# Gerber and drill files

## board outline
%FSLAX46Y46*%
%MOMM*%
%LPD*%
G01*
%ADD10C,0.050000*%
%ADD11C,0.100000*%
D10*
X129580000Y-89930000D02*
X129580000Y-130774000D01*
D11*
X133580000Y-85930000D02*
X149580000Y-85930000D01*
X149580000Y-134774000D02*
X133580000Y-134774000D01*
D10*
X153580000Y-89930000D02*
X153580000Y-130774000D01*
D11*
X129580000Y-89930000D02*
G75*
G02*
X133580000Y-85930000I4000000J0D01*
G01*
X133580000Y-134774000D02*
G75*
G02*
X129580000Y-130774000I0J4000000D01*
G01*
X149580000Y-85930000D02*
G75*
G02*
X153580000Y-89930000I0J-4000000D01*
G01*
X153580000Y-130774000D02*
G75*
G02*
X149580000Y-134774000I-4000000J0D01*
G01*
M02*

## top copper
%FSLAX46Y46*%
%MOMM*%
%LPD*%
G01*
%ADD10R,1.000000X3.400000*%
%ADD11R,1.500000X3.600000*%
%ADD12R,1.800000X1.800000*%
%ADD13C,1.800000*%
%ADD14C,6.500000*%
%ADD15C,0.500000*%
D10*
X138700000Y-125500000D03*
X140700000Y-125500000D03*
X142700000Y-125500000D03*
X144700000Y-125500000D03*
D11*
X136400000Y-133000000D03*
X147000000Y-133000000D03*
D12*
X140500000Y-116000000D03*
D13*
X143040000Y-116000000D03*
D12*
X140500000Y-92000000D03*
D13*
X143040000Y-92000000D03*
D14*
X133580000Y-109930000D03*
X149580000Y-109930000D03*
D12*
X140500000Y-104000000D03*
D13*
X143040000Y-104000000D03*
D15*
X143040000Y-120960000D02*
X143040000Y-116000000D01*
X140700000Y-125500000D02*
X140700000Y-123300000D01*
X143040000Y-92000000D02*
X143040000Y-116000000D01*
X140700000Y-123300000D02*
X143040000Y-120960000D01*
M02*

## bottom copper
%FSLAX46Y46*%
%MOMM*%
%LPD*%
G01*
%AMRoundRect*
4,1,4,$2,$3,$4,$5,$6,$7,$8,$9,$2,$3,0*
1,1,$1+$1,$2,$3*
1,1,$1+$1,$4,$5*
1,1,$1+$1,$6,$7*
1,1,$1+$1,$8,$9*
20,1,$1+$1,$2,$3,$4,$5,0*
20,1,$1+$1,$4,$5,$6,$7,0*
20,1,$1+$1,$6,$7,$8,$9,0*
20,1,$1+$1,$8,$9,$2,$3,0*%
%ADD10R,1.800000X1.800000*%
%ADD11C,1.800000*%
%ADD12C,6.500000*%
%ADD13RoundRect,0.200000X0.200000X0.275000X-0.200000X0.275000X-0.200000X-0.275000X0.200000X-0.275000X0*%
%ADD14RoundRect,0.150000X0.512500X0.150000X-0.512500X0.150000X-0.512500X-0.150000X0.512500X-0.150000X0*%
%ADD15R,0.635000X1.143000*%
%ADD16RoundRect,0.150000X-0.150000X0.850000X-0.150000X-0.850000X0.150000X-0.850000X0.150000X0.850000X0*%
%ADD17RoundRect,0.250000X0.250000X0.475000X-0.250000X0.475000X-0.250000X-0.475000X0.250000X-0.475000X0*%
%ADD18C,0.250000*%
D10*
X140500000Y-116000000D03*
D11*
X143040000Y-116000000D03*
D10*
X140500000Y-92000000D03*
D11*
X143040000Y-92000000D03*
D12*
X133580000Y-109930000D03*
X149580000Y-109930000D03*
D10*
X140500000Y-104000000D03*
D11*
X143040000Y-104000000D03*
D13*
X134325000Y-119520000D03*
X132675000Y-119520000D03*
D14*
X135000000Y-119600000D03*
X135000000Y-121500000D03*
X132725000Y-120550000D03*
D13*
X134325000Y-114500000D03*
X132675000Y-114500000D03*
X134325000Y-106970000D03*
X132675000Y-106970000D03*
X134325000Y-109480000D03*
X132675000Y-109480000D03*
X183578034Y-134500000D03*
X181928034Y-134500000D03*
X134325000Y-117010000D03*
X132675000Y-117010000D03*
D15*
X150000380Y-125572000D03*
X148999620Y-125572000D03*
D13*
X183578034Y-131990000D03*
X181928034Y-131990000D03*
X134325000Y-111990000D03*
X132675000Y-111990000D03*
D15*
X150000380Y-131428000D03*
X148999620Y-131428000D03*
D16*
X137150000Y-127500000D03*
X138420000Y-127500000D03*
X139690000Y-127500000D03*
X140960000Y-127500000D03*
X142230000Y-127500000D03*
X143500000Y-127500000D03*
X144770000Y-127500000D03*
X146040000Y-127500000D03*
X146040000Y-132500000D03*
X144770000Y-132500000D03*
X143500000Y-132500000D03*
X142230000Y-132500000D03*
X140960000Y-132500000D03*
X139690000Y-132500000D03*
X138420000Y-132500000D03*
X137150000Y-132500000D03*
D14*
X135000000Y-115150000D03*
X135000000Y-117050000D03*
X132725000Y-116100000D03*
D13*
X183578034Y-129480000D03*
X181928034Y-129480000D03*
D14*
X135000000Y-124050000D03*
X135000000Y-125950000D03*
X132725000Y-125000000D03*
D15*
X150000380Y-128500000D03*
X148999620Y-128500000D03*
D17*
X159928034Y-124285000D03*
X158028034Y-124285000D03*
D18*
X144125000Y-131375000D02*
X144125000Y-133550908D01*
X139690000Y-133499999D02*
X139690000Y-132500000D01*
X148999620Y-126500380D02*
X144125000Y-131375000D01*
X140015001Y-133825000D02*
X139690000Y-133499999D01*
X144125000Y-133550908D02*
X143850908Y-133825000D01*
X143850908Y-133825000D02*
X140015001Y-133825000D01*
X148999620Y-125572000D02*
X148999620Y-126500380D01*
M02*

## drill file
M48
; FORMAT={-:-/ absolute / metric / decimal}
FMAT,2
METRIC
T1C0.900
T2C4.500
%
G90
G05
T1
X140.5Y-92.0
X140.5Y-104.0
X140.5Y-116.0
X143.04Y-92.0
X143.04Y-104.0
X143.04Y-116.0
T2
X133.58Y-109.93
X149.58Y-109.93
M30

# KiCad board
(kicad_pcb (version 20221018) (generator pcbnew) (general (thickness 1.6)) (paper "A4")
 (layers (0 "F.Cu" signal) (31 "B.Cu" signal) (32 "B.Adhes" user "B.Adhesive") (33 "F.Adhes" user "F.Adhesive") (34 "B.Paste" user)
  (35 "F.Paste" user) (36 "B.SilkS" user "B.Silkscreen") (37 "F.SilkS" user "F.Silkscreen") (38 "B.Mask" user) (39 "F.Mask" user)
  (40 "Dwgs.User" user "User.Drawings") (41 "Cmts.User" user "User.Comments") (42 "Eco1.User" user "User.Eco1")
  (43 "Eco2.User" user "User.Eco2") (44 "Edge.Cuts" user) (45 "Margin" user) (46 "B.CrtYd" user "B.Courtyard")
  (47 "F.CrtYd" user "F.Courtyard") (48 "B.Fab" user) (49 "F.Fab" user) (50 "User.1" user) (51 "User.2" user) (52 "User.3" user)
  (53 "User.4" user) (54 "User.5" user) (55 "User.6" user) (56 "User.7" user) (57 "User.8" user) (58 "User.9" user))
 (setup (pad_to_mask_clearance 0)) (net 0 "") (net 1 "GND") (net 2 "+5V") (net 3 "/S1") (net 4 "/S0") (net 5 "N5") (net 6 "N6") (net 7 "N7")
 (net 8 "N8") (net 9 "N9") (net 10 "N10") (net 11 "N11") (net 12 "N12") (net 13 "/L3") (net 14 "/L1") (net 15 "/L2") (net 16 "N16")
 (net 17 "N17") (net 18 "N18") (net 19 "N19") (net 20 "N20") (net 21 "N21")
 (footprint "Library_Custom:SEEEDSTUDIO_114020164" (layer "F.Cu") (at 141.7 129.825)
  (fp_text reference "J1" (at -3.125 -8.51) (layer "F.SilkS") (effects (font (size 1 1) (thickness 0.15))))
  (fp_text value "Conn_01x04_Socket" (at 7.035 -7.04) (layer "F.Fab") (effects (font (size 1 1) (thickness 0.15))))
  (pad "1" smd rect (at -3 -4.325) (size 1 3.4) (layers "F.Cu" "F.Paste" "F.Mask") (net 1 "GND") (solder_mask_margin 0.102))
  (pad "2" smd rect (at -1 -4.325) (size 1 3.4) (layers "F.Cu" "F.Paste" "F.Mask") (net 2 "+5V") (solder_mask_margin 0.102))
  (pad "3" smd rect (at 1 -4.325) (size 1 3.4) (layers "F.Cu" "F.Paste" "F.Mask") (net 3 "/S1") (solder_mask_margin 0.102))
  (pad "4" smd rect (at 3 -4.325) (size 1 3.4) (layers "F.Cu" "F.Paste" "F.Mask") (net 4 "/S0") (solder_mask_margin 0.102))
  (pad "SH1" smd rect (at -5.3 3.175) (size 1.5 3.6) (layers "F.Cu" "F.Paste" "F.Mask") (solder_mask_margin 0.102))
  (pad "SH2" smd rect (at 5.3 3.175) (size 1.5 3.6) (layers "F.Cu" "F.Paste" "F.Mask") (solder_mask_margin 0.102)))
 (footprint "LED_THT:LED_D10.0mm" (layer "F.Cu") (at 140.5 116)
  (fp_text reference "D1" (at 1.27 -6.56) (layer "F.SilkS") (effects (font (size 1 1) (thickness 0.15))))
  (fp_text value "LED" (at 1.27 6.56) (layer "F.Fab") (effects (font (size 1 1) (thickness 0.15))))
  (pad "1" thru_hole rect (at 0 0) (size 1.8 1.8) (drill 0.9) (layers "*.Cu" "*.Mask") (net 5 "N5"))
  (pad "2" thru_hole circle (at 2.54 0) (size 1.8 1.8) (drill 0.9) (layers "*.Cu" "*.Mask") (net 2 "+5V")))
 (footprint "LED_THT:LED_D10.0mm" (layer "F.Cu") (at 140.5 92)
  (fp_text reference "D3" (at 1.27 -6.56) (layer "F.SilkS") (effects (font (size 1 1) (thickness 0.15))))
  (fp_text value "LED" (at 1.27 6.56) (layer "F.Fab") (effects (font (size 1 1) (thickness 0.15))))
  (pad "1" thru_hole rect (at 0 0) (size 1.8 1.8) (drill 0.9) (layers "*.Cu" "*.Mask") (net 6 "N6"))
  (pad "2" thru_hole circle (at 2.54 0) (size 1.8 1.8) (drill 0.9) (layers "*.Cu" "*.Mask") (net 2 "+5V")))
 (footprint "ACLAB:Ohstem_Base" (layer "F.Cu") (at 142.5 116)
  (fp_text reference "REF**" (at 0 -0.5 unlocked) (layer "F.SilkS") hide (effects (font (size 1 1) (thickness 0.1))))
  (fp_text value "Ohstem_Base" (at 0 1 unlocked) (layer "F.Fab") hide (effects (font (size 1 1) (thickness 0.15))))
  (fp_line (start -12.92 -26.07) (end -12.92 14.774) (stroke (width 0.05) (type default)) (layer "Edge.Cuts"))
  (fp_line (start -8.92 -30.07) (end 7.08 -30.07) (stroke (width 0.1) (type default)) (layer "Edge.Cuts"))
  (fp_line (start 7.08 18.774) (end -8.92 18.774) (stroke (width 0.1) (type default)) (layer "Edge.Cuts"))
  (fp_line (start 11.08 -26.07) (end 11.08 14.774) (stroke (width 0.05) (type default)) (layer "Edge.Cuts"))
  (fp_arc (start -12.92 -26.07) (mid -11.748427 -28.898427) (end -8.92 -30.07) (stroke (width 0.1) (type default)) (layer "Edge.Cuts"))
  (fp_arc (start -8.92 18.774) (mid -11.748427 17.602427) (end -12.92 14.774) (stroke (width 0.1) (type default)) (layer "Edge.Cuts"))
  (fp_arc (start 7.08 -30.07) (mid 9.908427 -28.898427) (end 11.08 -26.07) (stroke (width 0.1) (type default)) (layer "Edge.Cuts"))
  (fp_arc (start 11.08 14.774) (mid 9.908427 17.602427) (end 7.08 18.774) (stroke (width 0.1) (type default)) (layer "Edge.Cuts"))
  (pad "1" thru_hole circle (at -8.92 -6.07) (size 6.5 6.5) (drill 4.5) (layers "*.Cu" "*.Mask"))
  (pad "1" thru_hole circle (at 7.08 -6.07) (size 6.5 6.5) (drill 4.5) (layers "*.Cu" "*.Mask")))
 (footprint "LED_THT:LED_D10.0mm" (layer "F.Cu") (at 140.5 104)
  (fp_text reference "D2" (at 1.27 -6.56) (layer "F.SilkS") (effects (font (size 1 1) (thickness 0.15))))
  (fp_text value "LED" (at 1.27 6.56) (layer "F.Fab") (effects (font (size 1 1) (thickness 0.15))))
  (pad "1" thru_hole rect (at 0 0) (size 1.8 1.8) (drill 0.9) (layers "*.Cu" "*.Mask") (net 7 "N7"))
  (pad "2" thru_hole circle (at 2.54 0) (size 1.8 1.8) (drill 0.9) (layers "*.Cu" "*.Mask") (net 2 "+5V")))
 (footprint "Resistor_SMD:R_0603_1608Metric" (layer "B.Cu") (at 133.5 119.52 180)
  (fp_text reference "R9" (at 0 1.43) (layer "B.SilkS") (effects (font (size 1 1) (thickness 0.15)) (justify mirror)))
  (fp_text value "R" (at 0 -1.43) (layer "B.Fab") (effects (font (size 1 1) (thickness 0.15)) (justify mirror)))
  (pad "1" smd roundrect (at -0.825 0 180) (size 0.8 0.95) (layers "B.Cu" "B.Paste" "B.Mask") (roundrect_rratio 0.25) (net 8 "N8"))
  (pad "2" smd roundrect (at 0.825 0 180) (size 0.8 0.95) (layers "B.Cu" "B.Paste" "B.Mask") (roundrect_rratio 0.25) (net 1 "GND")))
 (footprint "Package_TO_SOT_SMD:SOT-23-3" (layer "B.Cu") (at 133.8625 120.55 180)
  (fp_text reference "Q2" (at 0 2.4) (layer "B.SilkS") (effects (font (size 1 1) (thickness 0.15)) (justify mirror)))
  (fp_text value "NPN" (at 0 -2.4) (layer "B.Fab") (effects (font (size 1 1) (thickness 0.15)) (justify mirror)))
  (pad "1" smd roundrect (at -1.1375 0.95 180) (size 1.325 0.6) (layers "B.Cu" "B.Paste" "B.Mask") (roundrect_rratio 0.25) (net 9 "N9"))
  (pad "2" smd roundrect (at -1.1375 -0.95 180) (size 1.325 0.6) (layers "B.Cu" "B.Paste" "B.Mask") (roundrect_rratio 0.25) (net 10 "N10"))
  (pad "3" smd roundrect (at 1.1375 0 180) (size 1.325 0.6) (layers "B.Cu" "B.Paste" "B.Mask") (roundrect_rratio 0.25) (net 1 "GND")))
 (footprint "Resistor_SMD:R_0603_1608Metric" (layer "B.Cu") (at 133.5 114.5 180)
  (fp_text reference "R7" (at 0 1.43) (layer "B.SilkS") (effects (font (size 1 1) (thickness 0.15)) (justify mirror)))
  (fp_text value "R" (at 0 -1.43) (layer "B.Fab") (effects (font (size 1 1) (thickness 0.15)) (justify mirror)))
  (pad "1" smd roundrect (at -0.825 0 180) (size 0.8 0.95) (layers "B.Cu" "B.Paste" "B.Mask") (roundrect_rratio 0.25) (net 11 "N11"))
  (pad "2" smd roundrect (at 0.825 0 180) (size 0.8 0.95) (layers "B.Cu" "B.Paste" "B.Mask") (roundrect_rratio 0.25) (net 1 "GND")))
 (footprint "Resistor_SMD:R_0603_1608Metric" (layer "B.Cu") (at 133.5 106.97 180)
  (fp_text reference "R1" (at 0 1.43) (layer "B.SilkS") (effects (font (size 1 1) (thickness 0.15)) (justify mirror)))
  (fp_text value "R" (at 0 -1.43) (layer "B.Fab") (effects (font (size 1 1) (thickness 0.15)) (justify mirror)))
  (pad "1" smd roundrect (at -0.825 0 180) (size 0.8 0.95) (layers "B.Cu" "B.Paste" "B.Mask") (roundrect_rratio 0.25) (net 5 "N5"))
  (pad "2" smd roundrect (at 0.825 0 180) (size 0.8 0.95) (layers "B.Cu" "B.Paste" "B.Mask") (roundrect_rratio 0.25) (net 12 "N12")))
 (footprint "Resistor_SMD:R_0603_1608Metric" (layer "B.Cu") (at 133.5 109.48 180)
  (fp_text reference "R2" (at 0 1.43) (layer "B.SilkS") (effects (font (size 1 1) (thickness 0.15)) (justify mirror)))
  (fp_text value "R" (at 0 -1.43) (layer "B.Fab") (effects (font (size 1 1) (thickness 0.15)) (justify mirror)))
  (pad "1" smd roundrect (at -0.825 0 180) (size 0.8 0.95) (layers "B.Cu" "B.Paste" "B.Mask") (roundrect_rratio 0.25) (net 7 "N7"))
  (pad "2" smd roundrect (at 0.825 0 180) (size 0.8 0.95) (layers "B.Cu" "B.Paste" "B.Mask") (roundrect_rratio 0.25) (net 9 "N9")))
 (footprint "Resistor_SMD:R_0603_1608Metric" (layer "B.Cu") (at 182.753034 134.5 180)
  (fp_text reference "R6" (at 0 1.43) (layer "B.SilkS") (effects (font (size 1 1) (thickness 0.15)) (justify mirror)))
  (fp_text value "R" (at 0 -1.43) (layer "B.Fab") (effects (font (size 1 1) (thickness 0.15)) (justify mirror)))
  (pad "1" smd roundrect (at -0.825 0 180) (size 0.8 0.95) (layers "B.Cu" "B.Paste" "B.Mask") (roundrect_rratio 0.25) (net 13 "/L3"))
  (pad "2" smd roundrect (at 0.825 0 180) (size 0.8 0.95) (layers "B.Cu" "B.Paste" "B.Mask") (roundrect_rratio 0.25) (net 8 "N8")))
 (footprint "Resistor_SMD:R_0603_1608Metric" (layer "B.Cu") (at 133.5 117.01 180)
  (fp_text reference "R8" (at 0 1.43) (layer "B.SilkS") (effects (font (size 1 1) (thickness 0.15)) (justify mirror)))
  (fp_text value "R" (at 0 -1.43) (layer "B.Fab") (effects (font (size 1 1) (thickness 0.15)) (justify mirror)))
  (pad "1" smd roundrect (at -0.825 0 180) (size 0.8 0.95) (layers "B.Cu" "B.Paste" "B.Mask") (roundrect_rratio 0.25) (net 10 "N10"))
  (pad "2" smd roundrect (at 0.825 0 180) (size 0.8 0.95) (layers "B.Cu" "B.Paste" "B.Mask") (roundrect_rratio 0.25) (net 1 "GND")))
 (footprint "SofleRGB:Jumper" (layer "B.Cu") (at 149.5 125.572 180)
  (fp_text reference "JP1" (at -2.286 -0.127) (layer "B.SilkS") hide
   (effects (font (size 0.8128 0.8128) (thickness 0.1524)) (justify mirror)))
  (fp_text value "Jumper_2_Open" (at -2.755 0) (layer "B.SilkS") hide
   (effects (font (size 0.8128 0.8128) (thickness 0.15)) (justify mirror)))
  (pad "1" smd rect (at -0.50038 0 180) (size 0.635 1.143) (layers "B.Cu" "B.Paste" "B.Mask") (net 12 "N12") (clearance 0.1905))
  (pad "2" smd rect (at 0.50038 0 180) (size 0.635 1.143) (layers "B.Cu" "B.Paste" "B.Mask") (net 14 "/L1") (clearance 0.1905)))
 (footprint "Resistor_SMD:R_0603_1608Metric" (layer "B.Cu") (at 182.753034 131.99 180)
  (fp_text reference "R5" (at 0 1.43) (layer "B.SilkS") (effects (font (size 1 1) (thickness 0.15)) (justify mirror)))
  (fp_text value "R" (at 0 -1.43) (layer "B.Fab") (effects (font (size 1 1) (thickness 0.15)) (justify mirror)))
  (pad "1" smd roundrect (at -0.825 0 180) (size 0.8 0.95) (layers "B.Cu" "B.Paste" "B.Mask") (roundrect_rratio 0.25) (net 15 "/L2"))
  (pad "2" smd roundrect (at 0.825 0 180) (size 0.8 0.95) (layers "B.Cu" "B.Paste" "B.Mask") (roundrect_rratio 0.25) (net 10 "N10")))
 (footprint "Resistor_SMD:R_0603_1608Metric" (layer "B.Cu") (at 133.5 111.99 180)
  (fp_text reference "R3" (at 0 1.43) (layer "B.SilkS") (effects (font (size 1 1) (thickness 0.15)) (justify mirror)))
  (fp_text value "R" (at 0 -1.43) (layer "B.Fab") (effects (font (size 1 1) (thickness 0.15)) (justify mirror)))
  (pad "1" smd roundrect (at -0.825 0 180) (size 0.8 0.95) (layers "B.Cu" "B.Paste" "B.Mask") (roundrect_rratio 0.25) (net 6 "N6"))
  (pad "2" smd roundrect (at 0.825 0 180) (size 0.8 0.95) (layers "B.Cu" "B.Paste" "B.Mask") (roundrect_rratio 0.25) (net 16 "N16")))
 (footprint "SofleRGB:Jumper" (layer "B.Cu") (at 149.5 131.428 180)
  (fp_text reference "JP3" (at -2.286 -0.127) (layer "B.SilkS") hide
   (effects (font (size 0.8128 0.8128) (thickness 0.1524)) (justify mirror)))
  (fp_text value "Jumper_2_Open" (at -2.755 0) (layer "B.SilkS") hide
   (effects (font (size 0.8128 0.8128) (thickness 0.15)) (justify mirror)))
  (pad "1" smd rect (at -0.50038 0 180) (size 0.635 1.143) (layers "B.Cu" "B.Paste" "B.Mask") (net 13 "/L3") (clearance 0.1905))
  (pad "2" smd rect (at 0.50038 0 180) (size 0.635 1.143) (layers "B.Cu" "B.Paste" "B.Mask") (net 16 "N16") (clearance 0.1905)))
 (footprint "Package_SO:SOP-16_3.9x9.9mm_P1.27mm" (layer "B.Cu") (at 141.595 130 -90)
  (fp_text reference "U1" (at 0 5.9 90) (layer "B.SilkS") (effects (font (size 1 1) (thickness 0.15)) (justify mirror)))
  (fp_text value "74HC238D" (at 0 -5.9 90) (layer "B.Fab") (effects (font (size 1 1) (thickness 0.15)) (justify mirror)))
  (pad "1" smd roundrect (at -2.5 4.445 270) (size 2 0.6) (layers "B.Cu" "B.Paste" "B.Mask") (roundrect_rratio 0.25) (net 4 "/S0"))
  (pad "2" smd roundrect (at -2.5 3.175 270) (size 2 0.6) (layers "B.Cu" "B.Paste" "B.Mask") (roundrect_rratio 0.25) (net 3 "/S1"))
  (pad "3" smd roundrect (at -2.5 1.905 270) (size 2 0.6) (layers "B.Cu" "B.Paste" "B.Mask") (roundrect_rratio 0.25) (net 1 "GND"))
  (pad "4" smd roundrect (at -2.5 0.635 270) (size 2 0.6) (layers "B.Cu" "B.Paste" "B.Mask") (roundrect_rratio 0.25) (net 1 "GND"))
  (pad "5" smd roundrect (at -2.5 -0.635 270) (size 2 0.6) (layers "B.Cu" "B.Paste" "B.Mask") (roundrect_rratio 0.25) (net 1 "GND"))
  (pad "6" smd roundrect (at -2.5 -1.905 270) (size 2 0.6) (layers "B.Cu" "B.Paste" "B.Mask") (roundrect_rratio 0.25) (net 2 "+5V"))
  (pad "7" smd roundrect (at -2.5 -3.175 270) (size 2 0.6) (layers "B.Cu" "B.Paste" "B.Mask") (roundrect_rratio 0.25) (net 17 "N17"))
  (pad "8" smd roundrect (at -2.5 -4.445 270) (size 2 0.6) (layers "B.Cu" "B.Paste" "B.Mask") (roundrect_rratio 0.25) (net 1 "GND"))
  (pad "9" smd roundrect (at 2.5 -4.445 270) (size 2 0.6) (layers "B.Cu" "B.Paste" "B.Mask") (roundrect_rratio 0.25) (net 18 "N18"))
  (pad "10" smd roundrect (at 2.5 -3.175 270) (size 2 0.6) (layers "B.Cu" "B.Paste" "B.Mask") (roundrect_rratio 0.25) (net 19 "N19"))
  (pad "11" smd roundrect (at 2.5 -1.905 270) (size 2 0.6) (layers "B.Cu" "B.Paste" "B.Mask") (roundrect_rratio 0.25) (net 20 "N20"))
  (pad "12" smd roundrect (at 2.5 -0.635 270) (size 2 0.6) (layers "B.Cu" "B.Paste" "B.Mask") (roundrect_rratio 0.25) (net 13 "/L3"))
  (pad "13" smd roundrect (at 2.5 0.635 270) (size 2 0.6) (layers "B.Cu" "B.Paste" "B.Mask") (roundrect_rratio 0.25) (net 15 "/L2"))
  (pad "14" smd roundrect (at 2.5 1.905 270) (size 2 0.6) (layers "B.Cu" "B.Paste" "B.Mask") (roundrect_rratio 0.25) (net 14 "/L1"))
  (pad "15" smd roundrect (at 2.5 3.175 270) (size 2 0.6) (layers "B.Cu" "B.Paste" "B.Mask") (roundrect_rratio 0.25) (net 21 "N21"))
  (pad "16" smd roundrect (at 2.5 4.445 270) (size 2 0.6) (layers "B.Cu" "B.Paste" "B.Mask") (roundrect_rratio 0.25) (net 2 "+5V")))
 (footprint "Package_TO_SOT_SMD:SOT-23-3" (layer "B.Cu") (at 133.8625 116.1 180)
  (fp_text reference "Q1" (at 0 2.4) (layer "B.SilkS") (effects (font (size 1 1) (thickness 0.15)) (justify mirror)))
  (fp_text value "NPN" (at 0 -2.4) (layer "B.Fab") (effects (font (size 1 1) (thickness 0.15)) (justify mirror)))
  (pad "1" smd roundrect (at -1.1375 0.95 180) (size 1.325 0.6) (layers "B.Cu" "B.Paste" "B.Mask") (roundrect_rratio 0.25) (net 12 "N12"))
  (pad "2" smd roundrect (at -1.1375 -0.95 180) (size 1.325 0.6) (layers "B.Cu" "B.Paste" "B.Mask") (roundrect_rratio 0.25) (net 11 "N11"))
  (pad "3" smd roundrect (at 1.1375 0 180) (size 1.325 0.6) (layers "B.Cu" "B.Paste" "B.Mask") (roundrect_rratio 0.25) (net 1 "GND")))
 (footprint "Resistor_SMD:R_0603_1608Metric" (layer "B.Cu") (at 182.753034 129.48 180)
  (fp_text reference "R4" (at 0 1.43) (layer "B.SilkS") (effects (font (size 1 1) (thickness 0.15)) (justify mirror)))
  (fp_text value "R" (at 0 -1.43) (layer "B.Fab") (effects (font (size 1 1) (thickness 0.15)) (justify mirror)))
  (pad "1" smd roundrect (at -0.825 0 180) (size 0.8 0.95) (layers "B.Cu" "B.Paste" "B.Mask") (roundrect_rratio 0.25) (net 14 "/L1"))
  (pad "2" smd roundrect (at 0.825 0 180) (size 0.8 0.95) (layers "B.Cu" "B.Paste" "B.Mask") (roundrect_rratio 0.25) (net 11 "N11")))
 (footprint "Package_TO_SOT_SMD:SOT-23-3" (layer "B.Cu") (at 133.8625 125 180)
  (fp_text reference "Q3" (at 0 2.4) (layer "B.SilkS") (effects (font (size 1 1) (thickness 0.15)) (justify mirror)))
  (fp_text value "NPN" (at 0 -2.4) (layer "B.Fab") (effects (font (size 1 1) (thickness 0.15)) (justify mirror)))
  (pad "1" smd roundrect (at -1.1375 0.95 180) (size 1.325 0.6) (layers "B.Cu" "B.Paste" "B.Mask") (roundrect_rratio 0.25) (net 16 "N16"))
  (pad "2" smd roundrect (at -1.1375 -0.95 180) (size 1.325 0.6) (layers "B.Cu" "B.Paste" "B.Mask") (roundrect_rratio 0.25) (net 8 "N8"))
  (pad "3" smd roundrect (at 1.1375 0 180) (size 1.325 0.6) (layers "B.Cu" "B.Paste" "B.Mask") (roundrect_rratio 0.25) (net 1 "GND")))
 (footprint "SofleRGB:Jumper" (layer "B.Cu") (at 149.5 128.5 180)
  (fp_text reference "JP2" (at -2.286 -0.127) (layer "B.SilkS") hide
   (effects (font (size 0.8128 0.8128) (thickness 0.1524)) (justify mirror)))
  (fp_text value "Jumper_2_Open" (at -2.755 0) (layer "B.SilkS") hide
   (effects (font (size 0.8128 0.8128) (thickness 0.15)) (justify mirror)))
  (pad "1" smd rect (at -0.50038 0 180) (size 0.635 1.143) (layers "B.Cu" "B.Paste" "B.Mask") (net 9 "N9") (clearance 0.1905))
  (pad "2" smd rect (at 0.50038 0 180) (size 0.635 1.143) (layers "B.Cu" "B.Paste" "B.Mask") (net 15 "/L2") (clearance 0.1905)))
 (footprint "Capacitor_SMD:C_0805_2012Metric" (layer "B.Cu") (at 158.978034 124.285 180)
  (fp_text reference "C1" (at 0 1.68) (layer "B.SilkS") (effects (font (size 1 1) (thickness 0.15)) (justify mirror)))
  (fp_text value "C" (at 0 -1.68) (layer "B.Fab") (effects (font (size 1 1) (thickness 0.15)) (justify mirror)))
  (pad "1" smd roundrect (at -0.95 0 180) (size 1 1.45) (layers "B.Cu" "B.Paste" "B.Mask") (roundrect_rratio 0.25) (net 2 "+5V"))
  (pad "2" smd roundrect (at 0.95 0 180) (size 1 1.45) (layers "B.Cu" "B.Paste" "B.Mask") (roundrect_rratio 0.25) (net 1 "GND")))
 (segment (start 143.04 120.96) (end 143.04 116) (width 0.5) (layer "F.Cu") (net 2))
 (segment (start 140.7 125.5) (end 140.7 123.3) (width 0.5) (layer "F.Cu") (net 2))
 (segment (start 143.04 92) (end 143.04 116) (width 0.5) (layer "F.Cu") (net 2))
 (segment (start 140.7 123.3) (end 143.04 120.96) (width 0.5) (layer "F.Cu") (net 2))
 (segment (start 144.125 131.375) (end 144.125 133.550908) (width 0.25) (layer "B.Cu") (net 14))
 (segment (start 139.69 133.499999) (end 139.69 132.5) (width 0.25) (layer "B.Cu") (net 14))
 (segment (start 148.99962 126.50038) (end 144.125 131.375) (width 0.25) (layer "B.Cu") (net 14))
 (segment (start 140.015001 133.825) (end 139.69 133.499999) (width 0.25) (layer "B.Cu") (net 14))
 (segment (start 144.125 133.550908) (end 143.850908 133.825) (width 0.25) (layer "B.Cu") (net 14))
 (segment (start 143.850908 133.825) (end 140.015001 133.825) (width 0.25) (layer "B.Cu") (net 14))
 (segment (start 148.99962 125.572) (end 148.99962 126.50038) (width 0.25) (layer "B.Cu") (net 14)))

